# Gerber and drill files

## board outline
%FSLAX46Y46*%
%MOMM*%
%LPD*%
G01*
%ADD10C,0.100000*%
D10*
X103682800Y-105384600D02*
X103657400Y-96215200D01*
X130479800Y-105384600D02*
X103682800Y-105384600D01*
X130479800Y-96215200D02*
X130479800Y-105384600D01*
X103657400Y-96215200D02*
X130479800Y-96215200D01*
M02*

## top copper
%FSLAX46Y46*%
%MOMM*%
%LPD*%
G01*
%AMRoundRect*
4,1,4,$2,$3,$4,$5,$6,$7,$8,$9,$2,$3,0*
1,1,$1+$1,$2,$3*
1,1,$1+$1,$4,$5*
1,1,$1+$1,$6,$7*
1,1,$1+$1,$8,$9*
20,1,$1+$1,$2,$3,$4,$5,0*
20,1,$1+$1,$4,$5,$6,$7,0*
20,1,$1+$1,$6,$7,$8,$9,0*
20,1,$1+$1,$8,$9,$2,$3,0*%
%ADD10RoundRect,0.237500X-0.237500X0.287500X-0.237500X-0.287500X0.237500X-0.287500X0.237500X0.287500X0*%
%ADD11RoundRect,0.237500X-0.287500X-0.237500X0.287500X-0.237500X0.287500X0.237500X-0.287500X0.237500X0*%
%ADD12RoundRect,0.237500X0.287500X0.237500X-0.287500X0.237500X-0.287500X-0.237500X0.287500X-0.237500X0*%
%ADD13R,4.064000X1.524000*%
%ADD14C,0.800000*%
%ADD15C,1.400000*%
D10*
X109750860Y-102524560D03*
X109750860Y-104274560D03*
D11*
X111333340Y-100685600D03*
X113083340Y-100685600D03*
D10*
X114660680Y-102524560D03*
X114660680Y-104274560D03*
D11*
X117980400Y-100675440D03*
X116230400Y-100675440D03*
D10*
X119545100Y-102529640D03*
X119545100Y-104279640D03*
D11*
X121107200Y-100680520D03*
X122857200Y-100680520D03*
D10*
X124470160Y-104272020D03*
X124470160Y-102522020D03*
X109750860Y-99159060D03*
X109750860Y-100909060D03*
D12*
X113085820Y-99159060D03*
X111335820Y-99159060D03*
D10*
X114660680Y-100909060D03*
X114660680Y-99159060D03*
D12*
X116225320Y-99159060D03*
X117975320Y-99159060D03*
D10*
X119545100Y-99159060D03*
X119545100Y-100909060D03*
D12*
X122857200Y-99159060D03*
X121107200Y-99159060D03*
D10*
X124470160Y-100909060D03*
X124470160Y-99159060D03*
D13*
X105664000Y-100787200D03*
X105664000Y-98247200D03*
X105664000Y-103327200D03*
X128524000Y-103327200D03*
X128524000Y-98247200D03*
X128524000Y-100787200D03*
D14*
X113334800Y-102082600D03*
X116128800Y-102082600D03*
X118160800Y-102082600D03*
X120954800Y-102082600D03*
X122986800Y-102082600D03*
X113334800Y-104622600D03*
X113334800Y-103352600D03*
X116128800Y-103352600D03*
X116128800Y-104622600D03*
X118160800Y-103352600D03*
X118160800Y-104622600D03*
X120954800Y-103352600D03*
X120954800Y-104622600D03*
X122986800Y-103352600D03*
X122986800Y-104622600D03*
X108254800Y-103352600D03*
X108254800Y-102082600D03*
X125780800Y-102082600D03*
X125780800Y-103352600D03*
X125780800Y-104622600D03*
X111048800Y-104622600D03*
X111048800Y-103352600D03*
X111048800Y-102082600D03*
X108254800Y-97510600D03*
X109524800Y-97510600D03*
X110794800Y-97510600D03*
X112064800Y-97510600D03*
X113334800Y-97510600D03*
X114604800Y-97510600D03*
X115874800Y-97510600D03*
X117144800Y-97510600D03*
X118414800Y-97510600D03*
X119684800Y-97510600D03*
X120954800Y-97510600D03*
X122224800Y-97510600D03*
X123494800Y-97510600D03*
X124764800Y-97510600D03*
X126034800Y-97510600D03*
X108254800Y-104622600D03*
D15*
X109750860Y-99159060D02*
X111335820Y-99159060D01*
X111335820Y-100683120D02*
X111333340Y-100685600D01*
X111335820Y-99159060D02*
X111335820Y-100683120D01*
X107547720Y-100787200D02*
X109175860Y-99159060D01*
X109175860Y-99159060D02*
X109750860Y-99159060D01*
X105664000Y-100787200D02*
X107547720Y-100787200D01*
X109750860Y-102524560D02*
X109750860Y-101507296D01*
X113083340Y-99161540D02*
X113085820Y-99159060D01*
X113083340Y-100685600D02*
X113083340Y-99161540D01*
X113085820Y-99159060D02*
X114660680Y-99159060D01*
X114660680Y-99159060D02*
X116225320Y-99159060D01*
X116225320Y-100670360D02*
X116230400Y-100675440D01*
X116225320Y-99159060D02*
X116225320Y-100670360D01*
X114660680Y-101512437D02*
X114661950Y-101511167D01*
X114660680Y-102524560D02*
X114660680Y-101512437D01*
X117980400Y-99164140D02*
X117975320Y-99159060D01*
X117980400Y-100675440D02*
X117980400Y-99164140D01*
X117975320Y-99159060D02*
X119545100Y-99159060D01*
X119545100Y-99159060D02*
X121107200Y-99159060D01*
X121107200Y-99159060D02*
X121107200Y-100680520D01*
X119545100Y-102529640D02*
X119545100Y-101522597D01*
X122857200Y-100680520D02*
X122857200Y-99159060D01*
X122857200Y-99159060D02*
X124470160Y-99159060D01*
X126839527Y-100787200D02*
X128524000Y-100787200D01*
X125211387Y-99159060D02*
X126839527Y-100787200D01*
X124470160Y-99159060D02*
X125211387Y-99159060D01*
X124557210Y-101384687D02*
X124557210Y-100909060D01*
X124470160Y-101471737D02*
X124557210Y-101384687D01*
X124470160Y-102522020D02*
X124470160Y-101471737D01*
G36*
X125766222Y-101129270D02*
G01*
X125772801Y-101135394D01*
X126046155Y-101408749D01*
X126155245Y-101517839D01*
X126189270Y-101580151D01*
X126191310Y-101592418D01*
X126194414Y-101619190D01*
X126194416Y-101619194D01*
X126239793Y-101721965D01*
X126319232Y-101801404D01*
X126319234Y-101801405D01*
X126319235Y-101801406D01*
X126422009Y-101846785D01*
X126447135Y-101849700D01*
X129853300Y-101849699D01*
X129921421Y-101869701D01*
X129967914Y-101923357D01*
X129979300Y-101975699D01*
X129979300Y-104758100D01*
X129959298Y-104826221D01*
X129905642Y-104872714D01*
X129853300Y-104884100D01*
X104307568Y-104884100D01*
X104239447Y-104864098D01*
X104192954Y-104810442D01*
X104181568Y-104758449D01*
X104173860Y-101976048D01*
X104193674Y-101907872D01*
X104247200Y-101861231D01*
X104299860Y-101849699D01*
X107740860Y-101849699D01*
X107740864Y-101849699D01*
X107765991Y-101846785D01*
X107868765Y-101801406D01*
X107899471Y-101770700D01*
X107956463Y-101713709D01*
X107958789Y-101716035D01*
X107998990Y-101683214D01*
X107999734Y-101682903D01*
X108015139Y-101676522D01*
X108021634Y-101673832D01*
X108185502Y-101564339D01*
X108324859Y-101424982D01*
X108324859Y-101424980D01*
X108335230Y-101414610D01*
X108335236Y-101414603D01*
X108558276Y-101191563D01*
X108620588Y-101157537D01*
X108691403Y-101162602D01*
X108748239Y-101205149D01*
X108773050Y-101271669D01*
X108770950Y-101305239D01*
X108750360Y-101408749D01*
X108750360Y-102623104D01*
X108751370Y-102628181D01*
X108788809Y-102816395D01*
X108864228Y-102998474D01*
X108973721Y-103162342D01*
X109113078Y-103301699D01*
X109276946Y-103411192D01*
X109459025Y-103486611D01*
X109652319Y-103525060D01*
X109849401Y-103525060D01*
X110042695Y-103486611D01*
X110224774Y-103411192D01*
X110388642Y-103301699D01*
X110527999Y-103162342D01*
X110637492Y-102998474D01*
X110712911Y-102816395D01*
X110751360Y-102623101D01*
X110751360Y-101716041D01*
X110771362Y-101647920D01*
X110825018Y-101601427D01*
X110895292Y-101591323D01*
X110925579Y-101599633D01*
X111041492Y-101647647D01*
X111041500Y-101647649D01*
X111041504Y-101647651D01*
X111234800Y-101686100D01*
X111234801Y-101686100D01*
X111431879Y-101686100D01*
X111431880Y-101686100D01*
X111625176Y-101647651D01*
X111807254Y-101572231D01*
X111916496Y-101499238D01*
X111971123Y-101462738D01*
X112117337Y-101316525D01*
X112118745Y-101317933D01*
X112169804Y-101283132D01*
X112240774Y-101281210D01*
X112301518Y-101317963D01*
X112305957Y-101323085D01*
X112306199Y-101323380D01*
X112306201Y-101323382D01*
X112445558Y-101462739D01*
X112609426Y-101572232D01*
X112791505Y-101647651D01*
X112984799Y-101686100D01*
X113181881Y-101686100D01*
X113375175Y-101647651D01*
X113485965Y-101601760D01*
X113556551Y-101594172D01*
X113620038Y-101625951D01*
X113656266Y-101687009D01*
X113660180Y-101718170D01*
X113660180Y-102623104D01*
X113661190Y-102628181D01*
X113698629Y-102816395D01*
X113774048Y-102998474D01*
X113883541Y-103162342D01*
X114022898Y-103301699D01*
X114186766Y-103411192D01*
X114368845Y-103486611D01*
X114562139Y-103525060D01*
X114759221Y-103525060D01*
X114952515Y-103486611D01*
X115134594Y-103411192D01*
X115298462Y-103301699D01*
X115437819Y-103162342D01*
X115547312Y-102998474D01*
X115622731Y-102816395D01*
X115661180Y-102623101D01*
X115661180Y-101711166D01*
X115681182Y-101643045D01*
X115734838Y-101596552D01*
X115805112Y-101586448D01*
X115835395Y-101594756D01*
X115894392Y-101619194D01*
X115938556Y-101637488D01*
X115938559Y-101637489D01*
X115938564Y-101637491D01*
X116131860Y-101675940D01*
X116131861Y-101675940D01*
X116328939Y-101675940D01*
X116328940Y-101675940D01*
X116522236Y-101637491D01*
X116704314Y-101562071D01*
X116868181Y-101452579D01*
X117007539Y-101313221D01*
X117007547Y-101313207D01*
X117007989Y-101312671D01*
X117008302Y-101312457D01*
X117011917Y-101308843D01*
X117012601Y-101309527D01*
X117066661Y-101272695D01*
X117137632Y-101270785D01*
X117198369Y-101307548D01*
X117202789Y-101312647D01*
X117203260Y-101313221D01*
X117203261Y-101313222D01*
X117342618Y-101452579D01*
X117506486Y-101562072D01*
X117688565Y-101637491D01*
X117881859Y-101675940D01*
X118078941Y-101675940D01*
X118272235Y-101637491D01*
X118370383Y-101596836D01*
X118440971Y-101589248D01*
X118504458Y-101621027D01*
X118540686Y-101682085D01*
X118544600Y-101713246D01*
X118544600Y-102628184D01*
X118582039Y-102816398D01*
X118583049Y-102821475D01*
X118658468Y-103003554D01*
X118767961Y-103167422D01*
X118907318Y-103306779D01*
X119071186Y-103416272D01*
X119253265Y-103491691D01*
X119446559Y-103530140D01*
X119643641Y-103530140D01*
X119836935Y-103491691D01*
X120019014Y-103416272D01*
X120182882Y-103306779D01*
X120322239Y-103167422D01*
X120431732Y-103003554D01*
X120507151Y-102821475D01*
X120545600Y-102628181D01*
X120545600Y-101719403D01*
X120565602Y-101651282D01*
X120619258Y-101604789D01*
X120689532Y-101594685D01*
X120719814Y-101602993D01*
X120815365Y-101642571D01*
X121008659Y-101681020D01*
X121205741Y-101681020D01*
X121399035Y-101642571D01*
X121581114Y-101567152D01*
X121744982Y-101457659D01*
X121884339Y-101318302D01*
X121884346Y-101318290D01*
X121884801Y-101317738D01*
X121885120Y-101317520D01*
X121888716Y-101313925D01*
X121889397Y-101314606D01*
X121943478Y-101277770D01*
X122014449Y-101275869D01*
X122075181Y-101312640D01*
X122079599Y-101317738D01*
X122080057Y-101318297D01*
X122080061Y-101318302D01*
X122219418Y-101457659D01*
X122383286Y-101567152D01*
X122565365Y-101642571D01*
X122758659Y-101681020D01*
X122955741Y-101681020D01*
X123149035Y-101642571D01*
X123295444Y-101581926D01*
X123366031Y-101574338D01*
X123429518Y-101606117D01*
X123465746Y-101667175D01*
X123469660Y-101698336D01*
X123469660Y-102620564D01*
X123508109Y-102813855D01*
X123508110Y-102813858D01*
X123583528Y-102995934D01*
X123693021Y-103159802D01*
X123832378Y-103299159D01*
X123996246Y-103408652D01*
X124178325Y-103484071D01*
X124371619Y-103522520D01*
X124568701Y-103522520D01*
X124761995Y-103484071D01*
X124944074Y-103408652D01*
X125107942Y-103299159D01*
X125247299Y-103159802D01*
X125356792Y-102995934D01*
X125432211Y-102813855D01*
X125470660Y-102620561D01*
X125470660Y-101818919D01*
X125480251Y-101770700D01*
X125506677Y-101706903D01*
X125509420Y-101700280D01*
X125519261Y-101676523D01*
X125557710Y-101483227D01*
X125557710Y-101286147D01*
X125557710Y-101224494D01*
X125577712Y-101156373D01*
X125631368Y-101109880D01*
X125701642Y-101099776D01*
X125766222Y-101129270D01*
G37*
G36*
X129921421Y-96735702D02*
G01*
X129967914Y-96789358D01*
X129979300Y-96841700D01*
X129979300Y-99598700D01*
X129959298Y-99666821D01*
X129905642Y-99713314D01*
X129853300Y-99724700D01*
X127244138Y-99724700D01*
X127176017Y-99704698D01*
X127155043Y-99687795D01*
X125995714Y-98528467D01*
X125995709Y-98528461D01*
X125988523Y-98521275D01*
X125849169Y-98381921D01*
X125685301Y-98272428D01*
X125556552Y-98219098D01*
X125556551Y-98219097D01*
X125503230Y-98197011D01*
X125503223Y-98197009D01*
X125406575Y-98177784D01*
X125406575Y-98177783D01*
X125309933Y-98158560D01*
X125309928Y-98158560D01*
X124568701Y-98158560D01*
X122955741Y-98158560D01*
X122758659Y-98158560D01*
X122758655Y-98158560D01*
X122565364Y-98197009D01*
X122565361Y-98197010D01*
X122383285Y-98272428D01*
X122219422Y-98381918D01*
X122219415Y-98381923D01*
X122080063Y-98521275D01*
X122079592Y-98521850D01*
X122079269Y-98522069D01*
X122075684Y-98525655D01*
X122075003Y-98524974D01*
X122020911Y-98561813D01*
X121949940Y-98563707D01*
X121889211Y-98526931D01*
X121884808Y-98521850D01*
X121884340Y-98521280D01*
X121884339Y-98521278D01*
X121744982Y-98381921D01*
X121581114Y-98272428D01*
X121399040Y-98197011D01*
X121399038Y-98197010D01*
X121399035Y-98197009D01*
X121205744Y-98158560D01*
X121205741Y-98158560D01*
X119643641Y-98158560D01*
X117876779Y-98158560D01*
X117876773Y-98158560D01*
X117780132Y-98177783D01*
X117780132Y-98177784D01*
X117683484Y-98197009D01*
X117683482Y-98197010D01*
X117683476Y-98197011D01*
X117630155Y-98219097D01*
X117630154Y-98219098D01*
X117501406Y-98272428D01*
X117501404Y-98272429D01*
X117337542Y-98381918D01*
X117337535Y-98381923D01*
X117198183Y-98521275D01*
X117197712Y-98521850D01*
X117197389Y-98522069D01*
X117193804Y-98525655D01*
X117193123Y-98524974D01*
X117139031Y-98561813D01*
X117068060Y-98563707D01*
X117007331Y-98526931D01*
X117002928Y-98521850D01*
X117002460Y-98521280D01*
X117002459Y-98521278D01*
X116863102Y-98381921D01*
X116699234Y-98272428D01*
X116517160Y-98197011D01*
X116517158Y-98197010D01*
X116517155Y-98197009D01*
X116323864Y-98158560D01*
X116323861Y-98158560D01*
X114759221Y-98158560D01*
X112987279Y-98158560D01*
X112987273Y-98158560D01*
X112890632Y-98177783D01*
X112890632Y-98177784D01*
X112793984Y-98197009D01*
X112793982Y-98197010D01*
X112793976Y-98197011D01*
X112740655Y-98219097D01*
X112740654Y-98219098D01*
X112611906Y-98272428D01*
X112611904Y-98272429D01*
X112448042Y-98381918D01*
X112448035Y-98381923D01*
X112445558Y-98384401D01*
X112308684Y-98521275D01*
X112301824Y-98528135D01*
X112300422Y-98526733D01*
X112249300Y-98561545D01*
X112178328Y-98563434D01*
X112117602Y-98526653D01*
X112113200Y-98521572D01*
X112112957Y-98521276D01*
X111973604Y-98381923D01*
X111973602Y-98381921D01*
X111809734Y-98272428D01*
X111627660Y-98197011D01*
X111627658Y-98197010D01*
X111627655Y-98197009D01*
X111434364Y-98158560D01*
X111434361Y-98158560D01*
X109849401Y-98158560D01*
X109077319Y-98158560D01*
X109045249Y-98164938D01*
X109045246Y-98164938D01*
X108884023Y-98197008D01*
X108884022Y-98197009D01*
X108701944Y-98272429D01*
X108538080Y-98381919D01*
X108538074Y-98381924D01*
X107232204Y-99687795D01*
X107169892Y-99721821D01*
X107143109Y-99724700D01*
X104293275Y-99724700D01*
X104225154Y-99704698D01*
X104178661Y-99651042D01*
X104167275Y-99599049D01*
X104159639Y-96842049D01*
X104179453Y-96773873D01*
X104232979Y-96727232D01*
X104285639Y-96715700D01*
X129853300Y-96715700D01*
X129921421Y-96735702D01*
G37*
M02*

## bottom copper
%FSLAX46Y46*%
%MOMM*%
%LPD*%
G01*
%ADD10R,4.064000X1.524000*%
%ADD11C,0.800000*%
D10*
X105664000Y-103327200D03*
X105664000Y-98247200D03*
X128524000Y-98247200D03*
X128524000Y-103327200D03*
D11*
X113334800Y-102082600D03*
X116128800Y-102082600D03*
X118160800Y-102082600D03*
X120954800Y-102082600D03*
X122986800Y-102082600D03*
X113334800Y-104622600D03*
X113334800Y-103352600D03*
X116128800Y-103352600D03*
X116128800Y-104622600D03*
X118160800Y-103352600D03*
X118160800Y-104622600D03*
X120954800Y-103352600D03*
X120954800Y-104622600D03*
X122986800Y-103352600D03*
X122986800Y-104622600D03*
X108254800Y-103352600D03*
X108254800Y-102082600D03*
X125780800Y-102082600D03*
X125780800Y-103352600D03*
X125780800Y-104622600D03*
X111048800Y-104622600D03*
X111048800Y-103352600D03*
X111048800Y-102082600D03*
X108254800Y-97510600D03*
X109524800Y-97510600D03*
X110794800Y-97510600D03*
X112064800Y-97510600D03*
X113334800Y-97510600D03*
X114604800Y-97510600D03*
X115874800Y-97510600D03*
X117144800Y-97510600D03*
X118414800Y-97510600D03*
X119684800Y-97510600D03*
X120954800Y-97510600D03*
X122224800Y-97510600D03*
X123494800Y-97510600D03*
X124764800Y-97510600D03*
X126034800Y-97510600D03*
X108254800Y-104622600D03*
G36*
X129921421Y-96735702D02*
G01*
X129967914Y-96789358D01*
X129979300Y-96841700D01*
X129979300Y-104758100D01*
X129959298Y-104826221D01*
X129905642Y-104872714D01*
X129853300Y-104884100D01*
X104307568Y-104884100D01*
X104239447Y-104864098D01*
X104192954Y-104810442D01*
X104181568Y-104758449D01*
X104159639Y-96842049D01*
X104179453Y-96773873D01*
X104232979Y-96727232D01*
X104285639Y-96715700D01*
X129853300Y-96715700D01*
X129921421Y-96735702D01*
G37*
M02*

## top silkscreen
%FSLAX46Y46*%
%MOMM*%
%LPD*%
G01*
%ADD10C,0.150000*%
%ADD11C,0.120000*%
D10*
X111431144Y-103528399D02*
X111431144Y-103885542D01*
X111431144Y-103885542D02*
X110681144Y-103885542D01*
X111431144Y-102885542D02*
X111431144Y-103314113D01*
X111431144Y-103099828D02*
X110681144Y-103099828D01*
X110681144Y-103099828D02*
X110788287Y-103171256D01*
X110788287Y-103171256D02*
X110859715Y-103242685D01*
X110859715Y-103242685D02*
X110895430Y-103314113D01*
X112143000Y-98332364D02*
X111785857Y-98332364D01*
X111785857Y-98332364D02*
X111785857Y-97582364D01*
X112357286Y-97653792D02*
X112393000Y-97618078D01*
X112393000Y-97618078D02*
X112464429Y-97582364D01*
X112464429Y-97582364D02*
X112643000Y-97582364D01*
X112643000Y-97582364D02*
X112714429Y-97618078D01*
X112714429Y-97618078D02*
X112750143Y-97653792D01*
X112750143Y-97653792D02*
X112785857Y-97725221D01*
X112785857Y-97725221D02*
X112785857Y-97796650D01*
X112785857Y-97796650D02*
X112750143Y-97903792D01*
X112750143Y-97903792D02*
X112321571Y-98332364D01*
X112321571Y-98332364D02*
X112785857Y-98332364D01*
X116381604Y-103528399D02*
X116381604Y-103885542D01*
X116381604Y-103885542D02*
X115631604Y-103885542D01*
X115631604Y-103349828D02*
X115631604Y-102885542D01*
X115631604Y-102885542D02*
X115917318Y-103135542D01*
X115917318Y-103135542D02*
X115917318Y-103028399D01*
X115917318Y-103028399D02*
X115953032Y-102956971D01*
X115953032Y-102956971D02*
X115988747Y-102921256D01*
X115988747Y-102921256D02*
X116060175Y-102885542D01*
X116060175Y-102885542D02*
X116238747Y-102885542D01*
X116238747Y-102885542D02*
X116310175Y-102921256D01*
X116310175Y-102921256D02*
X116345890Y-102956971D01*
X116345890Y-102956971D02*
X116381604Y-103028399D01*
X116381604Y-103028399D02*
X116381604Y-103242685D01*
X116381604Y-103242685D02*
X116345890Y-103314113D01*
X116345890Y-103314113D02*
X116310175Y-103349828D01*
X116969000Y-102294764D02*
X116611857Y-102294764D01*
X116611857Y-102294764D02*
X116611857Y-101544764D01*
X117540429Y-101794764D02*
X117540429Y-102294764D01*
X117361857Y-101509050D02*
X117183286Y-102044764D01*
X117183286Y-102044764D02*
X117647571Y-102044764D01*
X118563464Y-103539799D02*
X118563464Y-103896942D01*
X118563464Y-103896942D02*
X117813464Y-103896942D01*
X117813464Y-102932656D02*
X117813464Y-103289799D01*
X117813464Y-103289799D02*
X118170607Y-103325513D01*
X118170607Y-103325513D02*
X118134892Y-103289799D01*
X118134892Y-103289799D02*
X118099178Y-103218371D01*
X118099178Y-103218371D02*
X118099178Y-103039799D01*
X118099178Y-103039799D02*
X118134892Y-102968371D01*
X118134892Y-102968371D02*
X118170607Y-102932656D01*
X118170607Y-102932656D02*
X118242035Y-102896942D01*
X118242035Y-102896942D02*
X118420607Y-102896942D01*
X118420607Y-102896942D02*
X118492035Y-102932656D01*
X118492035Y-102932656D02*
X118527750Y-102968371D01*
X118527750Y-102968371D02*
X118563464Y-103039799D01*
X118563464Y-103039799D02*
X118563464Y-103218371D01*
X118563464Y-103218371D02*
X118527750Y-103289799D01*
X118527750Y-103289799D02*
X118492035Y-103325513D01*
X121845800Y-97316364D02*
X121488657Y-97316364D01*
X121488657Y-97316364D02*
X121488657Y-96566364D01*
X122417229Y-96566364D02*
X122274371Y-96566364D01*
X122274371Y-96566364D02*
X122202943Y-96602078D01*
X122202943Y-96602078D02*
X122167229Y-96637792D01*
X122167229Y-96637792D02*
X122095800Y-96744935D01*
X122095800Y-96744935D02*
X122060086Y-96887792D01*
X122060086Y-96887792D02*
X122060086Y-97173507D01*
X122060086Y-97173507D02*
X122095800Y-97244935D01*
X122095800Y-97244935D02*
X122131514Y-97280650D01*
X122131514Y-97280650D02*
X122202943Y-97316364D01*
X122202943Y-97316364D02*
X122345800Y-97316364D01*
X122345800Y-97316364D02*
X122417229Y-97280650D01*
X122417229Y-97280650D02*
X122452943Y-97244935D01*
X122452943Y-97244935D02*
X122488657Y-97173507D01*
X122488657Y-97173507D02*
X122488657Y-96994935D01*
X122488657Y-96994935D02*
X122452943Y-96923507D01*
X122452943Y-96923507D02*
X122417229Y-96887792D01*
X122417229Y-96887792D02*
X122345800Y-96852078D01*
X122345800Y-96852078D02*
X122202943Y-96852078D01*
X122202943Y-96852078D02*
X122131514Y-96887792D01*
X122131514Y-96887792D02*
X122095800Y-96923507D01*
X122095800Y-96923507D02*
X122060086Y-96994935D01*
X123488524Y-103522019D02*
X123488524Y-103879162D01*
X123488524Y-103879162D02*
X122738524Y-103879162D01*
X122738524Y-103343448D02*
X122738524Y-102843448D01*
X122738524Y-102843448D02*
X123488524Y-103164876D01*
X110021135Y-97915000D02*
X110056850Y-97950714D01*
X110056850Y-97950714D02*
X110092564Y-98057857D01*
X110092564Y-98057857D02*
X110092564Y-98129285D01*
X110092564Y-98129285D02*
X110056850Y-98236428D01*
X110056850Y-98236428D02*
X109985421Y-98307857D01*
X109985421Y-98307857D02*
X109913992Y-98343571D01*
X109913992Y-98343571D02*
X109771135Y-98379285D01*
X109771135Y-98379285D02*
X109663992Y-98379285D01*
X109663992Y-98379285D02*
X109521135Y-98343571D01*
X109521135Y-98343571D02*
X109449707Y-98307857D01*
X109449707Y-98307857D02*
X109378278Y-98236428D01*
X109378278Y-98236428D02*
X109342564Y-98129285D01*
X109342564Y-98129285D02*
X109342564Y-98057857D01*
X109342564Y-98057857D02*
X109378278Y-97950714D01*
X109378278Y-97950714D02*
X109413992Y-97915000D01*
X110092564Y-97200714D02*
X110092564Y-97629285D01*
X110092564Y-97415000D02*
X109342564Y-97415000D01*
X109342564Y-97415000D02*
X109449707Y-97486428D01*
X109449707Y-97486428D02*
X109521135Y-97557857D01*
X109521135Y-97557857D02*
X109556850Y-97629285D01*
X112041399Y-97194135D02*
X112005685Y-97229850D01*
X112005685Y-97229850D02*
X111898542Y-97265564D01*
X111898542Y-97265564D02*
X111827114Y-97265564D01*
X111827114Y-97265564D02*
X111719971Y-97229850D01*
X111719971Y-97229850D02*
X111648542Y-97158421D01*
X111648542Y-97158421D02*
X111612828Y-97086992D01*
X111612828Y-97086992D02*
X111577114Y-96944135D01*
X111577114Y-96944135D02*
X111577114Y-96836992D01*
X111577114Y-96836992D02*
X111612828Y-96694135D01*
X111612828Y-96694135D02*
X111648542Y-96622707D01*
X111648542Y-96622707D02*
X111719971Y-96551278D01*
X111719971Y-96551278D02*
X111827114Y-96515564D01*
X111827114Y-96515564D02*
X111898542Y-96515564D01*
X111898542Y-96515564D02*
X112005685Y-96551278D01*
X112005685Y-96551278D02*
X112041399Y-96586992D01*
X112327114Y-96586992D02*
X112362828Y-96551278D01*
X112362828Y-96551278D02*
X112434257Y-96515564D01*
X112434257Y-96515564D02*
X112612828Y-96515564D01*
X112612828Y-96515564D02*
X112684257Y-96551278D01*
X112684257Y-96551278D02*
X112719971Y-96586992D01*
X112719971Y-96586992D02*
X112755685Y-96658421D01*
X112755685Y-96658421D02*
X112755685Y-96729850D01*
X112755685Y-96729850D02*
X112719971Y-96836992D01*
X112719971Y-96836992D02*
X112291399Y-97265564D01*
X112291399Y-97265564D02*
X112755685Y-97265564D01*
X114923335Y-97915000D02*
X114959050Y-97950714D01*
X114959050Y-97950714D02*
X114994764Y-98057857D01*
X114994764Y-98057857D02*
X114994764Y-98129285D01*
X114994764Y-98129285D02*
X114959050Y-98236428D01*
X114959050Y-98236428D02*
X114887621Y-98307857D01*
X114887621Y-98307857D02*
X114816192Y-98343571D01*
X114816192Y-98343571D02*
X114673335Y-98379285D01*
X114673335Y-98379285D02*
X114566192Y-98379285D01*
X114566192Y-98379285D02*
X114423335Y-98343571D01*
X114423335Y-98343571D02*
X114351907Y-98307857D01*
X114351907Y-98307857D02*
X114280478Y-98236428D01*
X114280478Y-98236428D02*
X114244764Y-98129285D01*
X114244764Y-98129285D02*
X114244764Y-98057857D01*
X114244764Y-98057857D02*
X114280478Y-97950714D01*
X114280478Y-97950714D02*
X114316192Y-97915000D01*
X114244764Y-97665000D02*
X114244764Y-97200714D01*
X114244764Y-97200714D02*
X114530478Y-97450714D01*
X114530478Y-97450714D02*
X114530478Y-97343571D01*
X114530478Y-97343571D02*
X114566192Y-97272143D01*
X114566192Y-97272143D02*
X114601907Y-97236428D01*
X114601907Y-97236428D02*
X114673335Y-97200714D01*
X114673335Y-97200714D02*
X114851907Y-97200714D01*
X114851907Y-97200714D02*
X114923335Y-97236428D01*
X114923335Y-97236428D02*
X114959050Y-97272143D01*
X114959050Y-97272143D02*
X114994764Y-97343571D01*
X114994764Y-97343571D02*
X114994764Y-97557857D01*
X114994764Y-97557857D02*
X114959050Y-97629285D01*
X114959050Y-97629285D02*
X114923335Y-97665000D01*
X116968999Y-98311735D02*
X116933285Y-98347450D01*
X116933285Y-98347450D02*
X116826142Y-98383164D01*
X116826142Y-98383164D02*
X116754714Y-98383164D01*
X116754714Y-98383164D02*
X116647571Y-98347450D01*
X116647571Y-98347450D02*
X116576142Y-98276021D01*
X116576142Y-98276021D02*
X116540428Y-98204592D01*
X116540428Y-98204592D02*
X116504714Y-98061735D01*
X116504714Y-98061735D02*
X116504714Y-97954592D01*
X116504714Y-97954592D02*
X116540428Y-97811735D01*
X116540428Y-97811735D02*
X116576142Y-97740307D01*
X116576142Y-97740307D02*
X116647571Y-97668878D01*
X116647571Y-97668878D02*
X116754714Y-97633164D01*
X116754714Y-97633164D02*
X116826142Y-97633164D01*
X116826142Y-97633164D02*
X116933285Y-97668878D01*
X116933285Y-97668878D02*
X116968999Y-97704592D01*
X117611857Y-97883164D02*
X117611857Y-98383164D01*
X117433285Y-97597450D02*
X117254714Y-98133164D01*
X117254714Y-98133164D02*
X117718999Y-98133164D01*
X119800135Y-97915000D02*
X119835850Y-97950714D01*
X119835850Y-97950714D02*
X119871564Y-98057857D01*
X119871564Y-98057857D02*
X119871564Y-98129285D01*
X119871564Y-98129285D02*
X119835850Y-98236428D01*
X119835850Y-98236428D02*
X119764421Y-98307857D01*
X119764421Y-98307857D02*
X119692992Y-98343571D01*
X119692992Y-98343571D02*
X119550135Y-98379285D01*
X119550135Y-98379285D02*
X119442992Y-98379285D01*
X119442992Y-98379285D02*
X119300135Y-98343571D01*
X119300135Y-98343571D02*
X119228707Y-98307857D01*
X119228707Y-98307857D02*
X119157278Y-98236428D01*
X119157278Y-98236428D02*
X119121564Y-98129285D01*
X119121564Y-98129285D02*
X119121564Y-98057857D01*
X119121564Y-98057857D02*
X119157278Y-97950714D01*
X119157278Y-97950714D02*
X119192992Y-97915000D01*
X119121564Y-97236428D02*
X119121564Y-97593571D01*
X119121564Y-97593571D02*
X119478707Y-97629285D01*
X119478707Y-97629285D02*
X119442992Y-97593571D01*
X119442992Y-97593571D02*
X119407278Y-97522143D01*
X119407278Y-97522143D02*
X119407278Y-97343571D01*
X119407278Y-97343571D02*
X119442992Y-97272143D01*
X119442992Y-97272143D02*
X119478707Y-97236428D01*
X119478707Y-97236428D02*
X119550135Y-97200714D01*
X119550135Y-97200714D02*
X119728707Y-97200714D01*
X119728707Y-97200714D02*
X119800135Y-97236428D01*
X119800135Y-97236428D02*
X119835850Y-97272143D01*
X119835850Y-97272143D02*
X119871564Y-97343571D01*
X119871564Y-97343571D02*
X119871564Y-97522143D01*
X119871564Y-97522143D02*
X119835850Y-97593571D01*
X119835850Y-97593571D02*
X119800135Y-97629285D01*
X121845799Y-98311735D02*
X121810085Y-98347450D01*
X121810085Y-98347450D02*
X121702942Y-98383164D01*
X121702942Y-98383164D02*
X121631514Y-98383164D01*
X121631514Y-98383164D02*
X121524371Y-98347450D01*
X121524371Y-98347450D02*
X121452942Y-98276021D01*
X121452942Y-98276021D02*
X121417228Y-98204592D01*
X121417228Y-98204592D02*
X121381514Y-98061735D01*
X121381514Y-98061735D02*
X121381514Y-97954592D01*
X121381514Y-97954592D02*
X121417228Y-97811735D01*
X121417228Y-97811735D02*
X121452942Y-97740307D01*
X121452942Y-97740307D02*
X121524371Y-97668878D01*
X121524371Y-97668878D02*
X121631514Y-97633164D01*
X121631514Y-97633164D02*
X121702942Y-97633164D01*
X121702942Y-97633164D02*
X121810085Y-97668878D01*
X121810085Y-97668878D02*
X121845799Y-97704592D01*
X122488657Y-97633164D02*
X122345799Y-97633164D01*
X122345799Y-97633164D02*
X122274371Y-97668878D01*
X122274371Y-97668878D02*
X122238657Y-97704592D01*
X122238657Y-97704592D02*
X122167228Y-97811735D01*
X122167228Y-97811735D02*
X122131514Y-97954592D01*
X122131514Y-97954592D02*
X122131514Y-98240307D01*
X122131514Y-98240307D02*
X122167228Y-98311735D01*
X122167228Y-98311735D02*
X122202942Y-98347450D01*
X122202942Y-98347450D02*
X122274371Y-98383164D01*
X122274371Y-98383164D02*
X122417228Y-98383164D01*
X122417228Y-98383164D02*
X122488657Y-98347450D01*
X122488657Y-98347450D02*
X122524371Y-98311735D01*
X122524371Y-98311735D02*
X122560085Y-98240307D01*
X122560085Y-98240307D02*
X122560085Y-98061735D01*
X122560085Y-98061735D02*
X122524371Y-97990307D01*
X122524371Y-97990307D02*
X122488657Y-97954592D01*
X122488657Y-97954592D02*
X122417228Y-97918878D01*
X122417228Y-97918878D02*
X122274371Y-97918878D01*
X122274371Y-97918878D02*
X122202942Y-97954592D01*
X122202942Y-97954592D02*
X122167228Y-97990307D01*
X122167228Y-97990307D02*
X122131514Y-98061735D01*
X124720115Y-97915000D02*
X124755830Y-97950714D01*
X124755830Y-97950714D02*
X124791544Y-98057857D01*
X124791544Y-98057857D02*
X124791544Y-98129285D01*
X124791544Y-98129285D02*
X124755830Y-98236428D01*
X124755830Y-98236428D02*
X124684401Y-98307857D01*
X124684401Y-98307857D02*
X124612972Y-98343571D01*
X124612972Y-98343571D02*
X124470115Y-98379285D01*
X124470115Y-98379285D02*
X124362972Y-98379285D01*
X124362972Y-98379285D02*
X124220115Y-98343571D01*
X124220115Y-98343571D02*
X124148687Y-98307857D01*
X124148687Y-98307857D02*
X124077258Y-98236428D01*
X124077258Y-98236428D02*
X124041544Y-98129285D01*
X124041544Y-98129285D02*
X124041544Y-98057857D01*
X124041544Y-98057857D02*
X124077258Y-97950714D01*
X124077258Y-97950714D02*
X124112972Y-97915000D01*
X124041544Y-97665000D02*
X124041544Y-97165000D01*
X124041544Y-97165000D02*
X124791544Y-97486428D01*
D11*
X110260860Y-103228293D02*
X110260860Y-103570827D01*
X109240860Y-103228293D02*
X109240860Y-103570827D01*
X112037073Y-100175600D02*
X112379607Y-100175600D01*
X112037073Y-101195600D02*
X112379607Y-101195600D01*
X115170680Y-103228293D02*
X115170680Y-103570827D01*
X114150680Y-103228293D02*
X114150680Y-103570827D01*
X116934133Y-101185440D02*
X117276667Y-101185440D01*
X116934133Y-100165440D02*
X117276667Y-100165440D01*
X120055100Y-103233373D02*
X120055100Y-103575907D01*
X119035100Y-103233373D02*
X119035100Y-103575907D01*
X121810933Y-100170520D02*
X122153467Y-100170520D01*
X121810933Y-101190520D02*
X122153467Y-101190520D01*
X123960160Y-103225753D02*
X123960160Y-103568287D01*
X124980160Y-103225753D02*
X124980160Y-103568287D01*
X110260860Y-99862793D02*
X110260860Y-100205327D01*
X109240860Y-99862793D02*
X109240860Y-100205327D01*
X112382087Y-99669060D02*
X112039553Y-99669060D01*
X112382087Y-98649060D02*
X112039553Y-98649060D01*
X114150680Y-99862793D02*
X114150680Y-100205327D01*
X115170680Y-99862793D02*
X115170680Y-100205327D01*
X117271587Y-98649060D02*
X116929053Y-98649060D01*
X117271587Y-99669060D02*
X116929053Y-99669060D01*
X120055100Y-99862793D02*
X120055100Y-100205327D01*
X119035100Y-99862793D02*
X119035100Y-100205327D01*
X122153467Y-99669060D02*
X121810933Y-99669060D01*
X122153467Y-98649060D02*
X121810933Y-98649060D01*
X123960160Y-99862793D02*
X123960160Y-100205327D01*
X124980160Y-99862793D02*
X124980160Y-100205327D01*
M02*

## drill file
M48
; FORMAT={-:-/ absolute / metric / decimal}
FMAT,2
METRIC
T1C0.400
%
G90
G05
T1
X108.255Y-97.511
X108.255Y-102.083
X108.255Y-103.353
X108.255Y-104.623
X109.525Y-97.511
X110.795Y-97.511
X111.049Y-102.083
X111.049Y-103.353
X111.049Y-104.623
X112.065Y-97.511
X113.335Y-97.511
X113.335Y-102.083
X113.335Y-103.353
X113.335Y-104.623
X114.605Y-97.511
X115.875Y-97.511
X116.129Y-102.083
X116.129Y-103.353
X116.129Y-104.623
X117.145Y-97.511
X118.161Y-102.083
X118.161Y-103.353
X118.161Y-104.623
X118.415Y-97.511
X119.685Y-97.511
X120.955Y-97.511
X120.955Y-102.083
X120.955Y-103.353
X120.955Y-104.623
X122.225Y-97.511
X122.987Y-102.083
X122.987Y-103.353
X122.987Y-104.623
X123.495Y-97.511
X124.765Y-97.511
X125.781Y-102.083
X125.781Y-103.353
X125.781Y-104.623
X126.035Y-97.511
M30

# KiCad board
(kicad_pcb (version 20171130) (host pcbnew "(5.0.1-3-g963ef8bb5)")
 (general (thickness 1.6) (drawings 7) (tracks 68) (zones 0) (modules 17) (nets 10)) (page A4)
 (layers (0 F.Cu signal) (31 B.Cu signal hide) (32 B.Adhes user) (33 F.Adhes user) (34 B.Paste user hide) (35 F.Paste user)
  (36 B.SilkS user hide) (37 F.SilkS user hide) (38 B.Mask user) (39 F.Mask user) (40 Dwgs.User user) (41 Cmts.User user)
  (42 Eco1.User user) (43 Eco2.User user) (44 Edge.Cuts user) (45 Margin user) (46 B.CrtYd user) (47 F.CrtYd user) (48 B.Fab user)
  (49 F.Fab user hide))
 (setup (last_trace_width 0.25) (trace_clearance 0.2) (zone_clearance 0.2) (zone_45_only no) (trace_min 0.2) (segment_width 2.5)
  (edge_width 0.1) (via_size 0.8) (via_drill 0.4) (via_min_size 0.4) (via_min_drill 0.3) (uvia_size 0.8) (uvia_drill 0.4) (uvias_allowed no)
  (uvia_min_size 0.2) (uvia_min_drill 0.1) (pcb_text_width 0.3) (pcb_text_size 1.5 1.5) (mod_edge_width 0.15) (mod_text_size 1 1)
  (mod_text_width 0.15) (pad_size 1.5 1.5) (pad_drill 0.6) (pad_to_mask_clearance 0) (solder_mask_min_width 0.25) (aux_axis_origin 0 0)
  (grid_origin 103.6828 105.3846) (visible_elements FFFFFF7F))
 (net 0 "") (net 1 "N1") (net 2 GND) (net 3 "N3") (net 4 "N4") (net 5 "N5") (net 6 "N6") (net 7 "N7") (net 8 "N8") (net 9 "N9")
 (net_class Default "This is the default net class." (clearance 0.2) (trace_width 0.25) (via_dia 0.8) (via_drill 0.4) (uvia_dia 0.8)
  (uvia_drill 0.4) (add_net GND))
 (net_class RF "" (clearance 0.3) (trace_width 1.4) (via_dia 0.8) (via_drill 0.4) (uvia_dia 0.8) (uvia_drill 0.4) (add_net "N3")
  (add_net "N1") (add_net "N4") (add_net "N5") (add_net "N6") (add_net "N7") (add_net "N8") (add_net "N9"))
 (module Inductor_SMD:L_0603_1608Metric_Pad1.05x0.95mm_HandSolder (layer F.Cu) (at 109.75086 103.39956 270)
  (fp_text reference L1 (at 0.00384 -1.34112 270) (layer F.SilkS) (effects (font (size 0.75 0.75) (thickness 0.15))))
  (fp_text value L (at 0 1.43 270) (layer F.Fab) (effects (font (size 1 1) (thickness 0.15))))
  (fp_line (start -0.171267 -0.51) (end 0.171267 -0.51) (layer F.SilkS) (width 0.12))
  (fp_line (start -0.171267 0.51) (end 0.171267 0.51) (layer F.SilkS) (width 0.12))
  (pad 1 smd roundrect (at -0.875 0 270) (size 1.05 0.95) (layers F.Cu F.Paste F.Mask) (roundrect_rratio 0.25) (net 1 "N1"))
  (pad 2 smd roundrect (at 0.875 0 270) (size 1.05 0.95) (layers F.Cu F.Paste F.Mask) (roundrect_rratio 0.25) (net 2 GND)))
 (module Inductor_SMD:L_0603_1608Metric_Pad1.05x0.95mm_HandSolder (layer F.Cu) (at 112.20834 100.6856)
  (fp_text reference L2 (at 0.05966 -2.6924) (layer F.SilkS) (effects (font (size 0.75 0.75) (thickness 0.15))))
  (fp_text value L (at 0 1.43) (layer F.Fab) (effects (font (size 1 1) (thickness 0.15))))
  (fp_line (start -0.171267 -0.51) (end 0.171267 -0.51) (layer F.SilkS) (width 0.12))
  (fp_line (start -0.171267 0.51) (end 0.171267 0.51) (layer F.SilkS) (width 0.12))
  (pad 1 smd roundrect (at -0.875 0) (size 1.05 0.95) (layers F.Cu F.Paste F.Mask) (roundrect_rratio 0.25) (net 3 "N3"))
  (pad 2 smd roundrect (at 0.875 0) (size 1.05 0.95) (layers F.Cu F.Paste F.Mask) (roundrect_rratio 0.25) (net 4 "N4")))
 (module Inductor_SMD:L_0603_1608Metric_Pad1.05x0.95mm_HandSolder (layer F.Cu) (at 114.66068 103.39956 270)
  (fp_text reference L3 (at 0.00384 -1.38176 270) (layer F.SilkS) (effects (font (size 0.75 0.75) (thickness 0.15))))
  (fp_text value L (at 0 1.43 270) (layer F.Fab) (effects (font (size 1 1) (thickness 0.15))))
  (fp_line (start -0.171267 -0.51) (end 0.171267 -0.51) (layer F.SilkS) (width 0.12))
  (fp_line (start -0.171267 0.51) (end 0.171267 0.51) (layer F.SilkS) (width 0.12))
  (pad 1 smd roundrect (at -0.875 0 270) (size 1.05 0.95) (layers F.Cu F.Paste F.Mask) (roundrect_rratio 0.25) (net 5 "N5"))
  (pad 2 smd roundrect (at 0.875 0 270) (size 1.05 0.95) (layers F.Cu F.Paste F.Mask) (roundrect_rratio 0.25) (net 2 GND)))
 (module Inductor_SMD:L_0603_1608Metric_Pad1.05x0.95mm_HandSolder (layer F.Cu) (at 117.1054 100.67544)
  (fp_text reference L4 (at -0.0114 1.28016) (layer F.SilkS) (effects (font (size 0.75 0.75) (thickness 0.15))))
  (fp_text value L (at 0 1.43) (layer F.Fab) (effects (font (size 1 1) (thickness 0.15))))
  (fp_line (start -0.171267 0.51) (end 0.171267 0.51) (layer F.SilkS) (width 0.12))
  (fp_line (start -0.171267 -0.51) (end 0.171267 -0.51) (layer F.SilkS) (width 0.12))
  (pad 2 smd roundrect (at 0.875 0) (size 1.05 0.95) (layers F.Cu F.Paste F.Mask) (roundrect_rratio 0.25) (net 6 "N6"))
  (pad 1 smd roundrect (at -0.875 0) (size 1.05 0.95) (layers F.Cu F.Paste F.Mask) (roundrect_rratio 0.25) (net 4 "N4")))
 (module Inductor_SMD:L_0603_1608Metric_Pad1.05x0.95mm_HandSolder (layer F.Cu) (at 119.5451 103.40464 270)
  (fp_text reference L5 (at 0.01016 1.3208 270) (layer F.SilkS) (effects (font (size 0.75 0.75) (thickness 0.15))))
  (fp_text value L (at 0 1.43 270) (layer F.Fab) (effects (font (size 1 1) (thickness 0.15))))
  (fp_line (start -0.171267 -0.51) (end 0.171267 -0.51) (layer F.SilkS) (width 0.12))
  (fp_line (start -0.171267 0.51) (end 0.171267 0.51) (layer F.SilkS) (width 0.12))
  (pad 1 smd roundrect (at -0.875 0 270) (size 1.05 0.95) (layers F.Cu F.Paste F.Mask) (roundrect_rratio 0.25) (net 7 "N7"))
  (pad 2 smd roundrect (at 0.875 0 270) (size 1.05 0.95) (layers F.Cu F.Paste F.Mask) (roundrect_rratio 0.25) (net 2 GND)))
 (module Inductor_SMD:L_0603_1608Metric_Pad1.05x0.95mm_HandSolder (layer F.Cu) (at 121.9822 100.68052)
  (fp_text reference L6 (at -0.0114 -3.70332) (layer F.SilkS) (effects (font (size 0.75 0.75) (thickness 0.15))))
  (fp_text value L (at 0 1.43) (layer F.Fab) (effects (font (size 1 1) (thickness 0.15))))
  (fp_line (start -0.171267 -0.51) (end 0.171267 -0.51) (layer F.SilkS) (width 0.12))
  (fp_line (start -0.171267 0.51) (end 0.171267 0.51) (layer F.SilkS) (width 0.12))
  (pad 1 smd roundrect (at -0.875 0) (size 1.05 0.95) (layers F.Cu F.Paste F.Mask) (roundrect_rratio 0.25) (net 6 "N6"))
  (pad 2 smd roundrect (at 0.875 0) (size 1.05 0.95) (layers F.Cu F.Paste F.Mask) (roundrect_rratio 0.25) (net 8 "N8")))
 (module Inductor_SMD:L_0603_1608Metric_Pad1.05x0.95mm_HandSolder (layer F.Cu) (at 124.47016 103.39702 270)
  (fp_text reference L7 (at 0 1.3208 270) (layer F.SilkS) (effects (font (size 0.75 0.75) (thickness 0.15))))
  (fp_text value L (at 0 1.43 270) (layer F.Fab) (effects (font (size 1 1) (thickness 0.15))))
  (fp_line (start -0.171267 0.51) (end 0.171267 0.51) (layer F.SilkS) (width 0.12))
  (fp_line (start -0.171267 -0.51) (end 0.171267 -0.51) (layer F.SilkS) (width 0.12))
  (pad 2 smd roundrect (at 0.875 0 270) (size 1.05 0.95) (layers F.Cu F.Paste F.Mask) (roundrect_rratio 0.25) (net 2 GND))
  (pad 1 smd roundrect (at -0.875 0 270) (size 1.05 0.95) (layers F.Cu F.Paste F.Mask) (roundrect_rratio 0.25) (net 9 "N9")))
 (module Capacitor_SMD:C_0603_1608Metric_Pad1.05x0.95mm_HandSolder (layer F.Cu) (at 109.75086 100.03406 270)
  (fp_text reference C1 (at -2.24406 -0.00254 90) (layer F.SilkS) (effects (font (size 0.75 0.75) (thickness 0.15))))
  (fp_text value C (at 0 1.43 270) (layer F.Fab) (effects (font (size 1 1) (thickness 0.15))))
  (fp_line (start -0.171267 -0.51) (end 0.171267 -0.51) (layer F.SilkS) (width 0.12))
  (fp_line (start -0.171267 0.51) (end 0.171267 0.51) (layer F.SilkS) (width 0.12))
  (pad 1 smd roundrect (at -0.875 0 270) (size 1.05 0.95) (layers F.Cu F.Paste F.Mask) (roundrect_rratio 0.25) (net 3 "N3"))
  (pad 2 smd roundrect (at 0.875 0 270) (size 1.05 0.95) (layers F.Cu F.Paste F.Mask) (roundrect_rratio 0.25) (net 1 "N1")))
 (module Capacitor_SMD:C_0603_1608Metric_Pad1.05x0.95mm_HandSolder (layer F.Cu) (at 112.21082 99.15906 180)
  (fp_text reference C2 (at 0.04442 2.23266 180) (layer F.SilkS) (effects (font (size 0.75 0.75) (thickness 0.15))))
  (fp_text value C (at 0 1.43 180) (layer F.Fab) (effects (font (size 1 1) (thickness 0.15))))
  (fp_line (start -0.171267 -0.51) (end 0.171267 -0.51) (layer F.SilkS) (width 0.12))
  (fp_line (start -0.171267 0.51) (end 0.171267 0.51) (layer F.SilkS) (width 0.12))
  (pad 1 smd roundrect (at -0.875 0 180) (size 1.05 0.95) (layers F.Cu F.Paste F.Mask) (roundrect_rratio 0.25) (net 4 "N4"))
  (pad 2 smd roundrect (at 0.875 0 180) (size 1.05 0.95) (layers F.Cu F.Paste F.Mask) (roundrect_rratio 0.25) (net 3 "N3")))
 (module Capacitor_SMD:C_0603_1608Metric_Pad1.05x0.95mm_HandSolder (layer F.Cu) (at 114.66068 100.03406 270)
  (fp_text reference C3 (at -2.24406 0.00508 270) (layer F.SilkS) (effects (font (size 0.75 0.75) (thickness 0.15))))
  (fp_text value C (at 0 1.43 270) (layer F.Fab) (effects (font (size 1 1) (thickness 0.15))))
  (fp_line (start -0.171267 0.51) (end 0.171267 0.51) (layer F.SilkS) (width 0.12))
  (fp_line (start -0.171267 -0.51) (end 0.171267 -0.51) (layer F.SilkS) (width 0.12))
  (pad 2 smd roundrect (at 0.875 0 270) (size 1.05 0.95) (layers F.Cu F.Paste F.Mask) (roundrect_rratio 0.25) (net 5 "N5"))
  (pad 1 smd roundrect (at -0.875 0 270) (size 1.05 0.95) (layers F.Cu F.Paste F.Mask) (roundrect_rratio 0.25) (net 4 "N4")))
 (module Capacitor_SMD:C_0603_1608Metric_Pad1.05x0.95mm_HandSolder (layer F.Cu) (at 117.10032 99.15906 180)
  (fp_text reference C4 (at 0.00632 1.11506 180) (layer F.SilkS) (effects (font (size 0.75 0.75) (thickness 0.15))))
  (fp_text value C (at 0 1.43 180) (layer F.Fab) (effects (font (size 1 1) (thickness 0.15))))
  (fp_line (start -0.171267 0.51) (end 0.171267 0.51) (layer F.SilkS) (width 0.12))
  (fp_line (start -0.171267 -0.51) (end 0.171267 -0.51) (layer F.SilkS) (width 0.12))
  (pad 2 smd roundrect (at 0.875 0 180) (size 1.05 0.95) (layers F.Cu F.Paste F.Mask) (roundrect_rratio 0.25) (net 4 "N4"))
  (pad 1 smd roundrect (at -0.875 0 180) (size 1.05 0.95) (layers F.Cu F.Paste F.Mask) (roundrect_rratio 0.25) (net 6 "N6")))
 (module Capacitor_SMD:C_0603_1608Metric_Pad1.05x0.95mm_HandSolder (layer F.Cu) (at 119.5451 100.03406 270)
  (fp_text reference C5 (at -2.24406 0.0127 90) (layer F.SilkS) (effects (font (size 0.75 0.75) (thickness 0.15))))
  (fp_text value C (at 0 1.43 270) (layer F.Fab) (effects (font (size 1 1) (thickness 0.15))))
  (fp_line (start -0.171267 -0.51) (end 0.171267 -0.51) (layer F.SilkS) (width 0.12))
  (fp_line (start -0.171267 0.51) (end 0.171267 0.51) (layer F.SilkS) (width 0.12))
  (pad 1 smd roundrect (at -0.875 0 270) (size 1.05 0.95) (layers F.Cu F.Paste F.Mask) (roundrect_rratio 0.25) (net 6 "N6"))
  (pad 2 smd roundrect (at 0.875 0 270) (size 1.05 0.95) (layers F.Cu F.Paste F.Mask) (roundrect_rratio 0.25) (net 7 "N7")))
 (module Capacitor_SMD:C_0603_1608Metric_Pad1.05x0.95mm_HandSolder (layer F.Cu) (at 121.9822 99.15906 180)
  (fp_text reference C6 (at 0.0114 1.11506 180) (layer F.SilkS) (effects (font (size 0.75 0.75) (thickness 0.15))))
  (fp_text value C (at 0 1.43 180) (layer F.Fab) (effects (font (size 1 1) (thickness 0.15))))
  (fp_line (start -0.171267 -0.51) (end 0.171267 -0.51) (layer F.SilkS) (width 0.12))
  (fp_line (start -0.171267 0.51) (end 0.171267 0.51) (layer F.SilkS) (width 0.12))
  (pad 1 smd roundrect (at -0.875 0 180) (size 1.05 0.95) (layers F.Cu F.Paste F.Mask) (roundrect_rratio 0.25) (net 8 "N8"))
  (pad 2 smd roundrect (at 0.875 0 180) (size 1.05 0.95) (layers F.Cu F.Paste F.Mask) (roundrect_rratio 0.25) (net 6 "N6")))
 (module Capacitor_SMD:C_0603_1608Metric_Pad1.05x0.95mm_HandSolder (layer F.Cu) (at 124.47016 100.03406 270)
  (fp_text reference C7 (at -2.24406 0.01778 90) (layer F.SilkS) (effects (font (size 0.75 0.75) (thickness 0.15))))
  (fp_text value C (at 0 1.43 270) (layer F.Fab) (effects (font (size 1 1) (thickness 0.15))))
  (fp_line (start -0.171267 0.51) (end 0.171267 0.51) (layer F.SilkS) (width 0.12))
  (fp_line (start -0.171267 -0.51) (end 0.171267 -0.51) (layer F.SilkS) (width 0.12))
  (pad 2 smd roundrect (at 0.875 0 270) (size 1.05 0.95) (layers F.Cu F.Paste F.Mask) (roundrect_rratio 0.25) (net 9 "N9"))
  (pad 1 smd roundrect (at -0.875 0 270) (size 1.05 0.95) (layers F.Cu F.Paste F.Mask) (roundrect_rratio 0.25) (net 8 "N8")))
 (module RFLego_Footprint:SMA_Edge (layer F.Cu) (at 103.632 100.7872)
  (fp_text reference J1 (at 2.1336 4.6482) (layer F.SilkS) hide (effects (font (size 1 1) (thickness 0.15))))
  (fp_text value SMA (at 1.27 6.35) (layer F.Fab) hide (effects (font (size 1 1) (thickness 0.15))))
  (pad 1 smd rect (at 2.032 0) (size 4.064 1.524) (layers F.Cu F.Mask) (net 3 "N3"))
  (pad 2 smd rect (at 2.032 -2.54) (size 4.064 1.524) (layers F.Cu F.Mask) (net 2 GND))
  (pad 2 smd rect (at 2.032 2.54) (size 4.064 1.524) (layers B.Cu B.Mask) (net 2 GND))
  (pad 2 smd rect (at 2.032 -2.54) (size 4.064 1.524) (layers B.Cu B.Mask) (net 2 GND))
  (pad 2 smd rect (at 2.032 2.54) (size 4.064 1.524) (layers F.Cu F.Mask) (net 2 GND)))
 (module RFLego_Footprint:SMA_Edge (layer F.Cu) (at 126.492 100.7872)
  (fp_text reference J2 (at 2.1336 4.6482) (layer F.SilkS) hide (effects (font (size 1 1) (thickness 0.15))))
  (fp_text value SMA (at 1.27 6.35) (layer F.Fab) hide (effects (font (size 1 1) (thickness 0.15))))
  (pad 2 smd rect (at 2.032 2.54) (size 4.064 1.524) (layers F.Cu F.Mask) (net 2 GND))
  (pad 2 smd rect (at 2.032 -2.54) (size 4.064 1.524) (layers B.Cu B.Mask) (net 2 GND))
  (pad 2 smd rect (at 2.032 2.54) (size 4.064 1.524) (layers B.Cu B.Mask) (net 2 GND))
  (pad 2 smd rect (at 2.032 -2.54) (size 4.064 1.524) (layers F.Cu F.Mask) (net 2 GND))
  (pad 1 smd rect (at 2.032 0) (size 4.064 1.524) (layers F.Cu F.Mask) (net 8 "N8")))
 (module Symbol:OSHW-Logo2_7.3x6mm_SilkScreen (layer B.Cu) (at 111.00816 102.235 180)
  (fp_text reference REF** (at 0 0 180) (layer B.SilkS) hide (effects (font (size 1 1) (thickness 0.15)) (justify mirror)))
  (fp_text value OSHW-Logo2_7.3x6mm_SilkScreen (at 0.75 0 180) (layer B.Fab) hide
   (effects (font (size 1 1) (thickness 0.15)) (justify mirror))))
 (gr_line (start 103.6828 105.3846) (end 103.6574 96.2152) (layer Edge.Cuts) (width 0.1))
 (gr_line (start 130.4798 105.3846) (end 103.6828 105.3846) (layer Edge.Cuts) (width 0.1))
 (gr_line (start 130.4798 96.2152) (end 130.4798 105.3846) (layer Edge.Cuts) (width 0.1))
 (gr_line (start 103.6574 96.2152) (end 130.4798 96.2152) (layer Edge.Cuts) (width 0.1))
 (via (at 113.3348 102.0826) (size 0.8) (drill 0.4) (layers F.Cu B.Cu) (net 2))
 (via (at 116.1288 102.0826) (size 0.8) (drill 0.4) (layers F.Cu B.Cu) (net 2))
 (via (at 118.1608 102.0826) (size 0.8) (drill 0.4) (layers F.Cu B.Cu) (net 2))
 (via (at 120.9548 102.0826) (size 0.8) (drill 0.4) (layers F.Cu B.Cu) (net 2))
 (via (at 122.9868 102.0826) (size 0.8) (drill 0.4) (layers F.Cu B.Cu) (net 2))
 (via (at 113.3348 104.6226) (size 0.8) (drill 0.4) (layers F.Cu B.Cu) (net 2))
 (via (at 113.3348 103.3526) (size 0.8) (drill 0.4) (layers F.Cu B.Cu) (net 2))
 (via (at 116.1288 103.3526) (size 0.8) (drill 0.4) (layers F.Cu B.Cu) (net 2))
 (via (at 116.1288 104.6226) (size 0.8) (drill 0.4) (layers F.Cu B.Cu) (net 2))
 (via (at 118.1608 103.3526) (size 0.8) (drill 0.4) (layers F.Cu B.Cu) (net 2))
 (via (at 118.1608 104.6226) (size 0.8) (drill 0.4) (layers F.Cu B.Cu) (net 2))
 (via (at 120.9548 103.3526) (size 0.8) (drill 0.4) (layers F.Cu B.Cu) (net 2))
 (via (at 120.9548 104.6226) (size 0.8) (drill 0.4) (layers F.Cu B.Cu) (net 2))
 (via (at 122.9868 103.3526) (size 0.8) (drill 0.4) (layers F.Cu B.Cu) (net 2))
 (via (at 122.9868 104.6226) (size 0.8) (drill 0.4) (layers F.Cu B.Cu) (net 2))
 (via (at 108.2548 103.3526) (size 0.8) (drill 0.4) (layers F.Cu B.Cu) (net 2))
 (via (at 108.2548 102.0826) (size 0.8) (drill 0.4) (layers F.Cu B.Cu) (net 2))
 (via (at 125.7808 102.0826) (size 0.8) (drill 0.4) (layers F.Cu B.Cu) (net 2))
 (via (at 125.7808 103.3526) (size 0.8) (drill 0.4) (layers F.Cu B.Cu) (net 2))
 (via (at 125.7808 104.6226) (size 0.8) (drill 0.4) (layers F.Cu B.Cu) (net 2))
 (via (at 111.0488 104.6226) (size 0.8) (drill 0.4) (layers F.Cu B.Cu) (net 2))
 (via (at 111.0488 103.3526) (size 0.8) (drill 0.4) (layers F.Cu B.Cu) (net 2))
 (via (at 111.0488 102.0826) (size 0.8) (drill 0.4) (layers F.Cu B.Cu) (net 2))
 (segment (start 109.75086 99.15906) (end 111.33582 99.15906) (width 1.4) (layer F.Cu) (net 3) (status 30))
 (segment (start 111.33582 100.68312) (end 111.33334 100.6856) (width 1.4) (layer F.Cu) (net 3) (status 30))
 (segment (start 111.33582 99.15906) (end 111.33582 100.68312) (width 1.4) (layer F.Cu) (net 3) (status 30))
 (segment (start 107.54772 100.7872) (end 109.17586 99.15906) (width 1.4) (layer F.Cu) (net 3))
 (segment (start 109.17586 99.15906) (end 109.75086 99.15906) (width 1.4) (layer F.Cu) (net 3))
 (segment (start 105.664 100.7872) (end 107.54772 100.7872) (width 1.4) (layer F.Cu) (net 3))
 (segment (start 109.75086 102.52456) (end 109.75086 101.507296) (width 1.4) (layer F.Cu) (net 1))
 (segment (start 113.08334 99.16154) (end 113.08582 99.15906) (width 1.4) (layer F.Cu) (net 4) (status 30))
 (segment (start 113.08334 100.6856) (end 113.08334 99.16154) (width 1.4) (layer F.Cu) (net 4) (status 30))
 (segment (start 113.08582 99.15906) (end 114.66068 99.15906) (width 1.4) (layer F.Cu) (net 4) (status 30))
 (segment (start 114.66068 99.15906) (end 116.22532 99.15906) (width 1.4) (layer F.Cu) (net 4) (status 30))
 (segment (start 116.22532 100.67036) (end 116.2304 100.67544) (width 1.4) (layer F.Cu) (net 4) (status 30))
 (segment (start 116.22532 99.15906) (end 116.22532 100.67036) (width 1.4) (layer F.Cu) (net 4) (status 30))
 (segment (start 114.66068 101.512437) (end 114.66195 101.511167) (width 1.4) (layer F.Cu) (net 5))
 (segment (start 114.66068 102.52456) (end 114.66068 101.512437) (width 1.4) (layer F.Cu) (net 5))
 (segment (start 117.9804 99.16414) (end 117.97532 99.15906) (width 1.4) (layer F.Cu) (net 6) (status 30))
 (segment (start 117.9804 100.67544) (end 117.9804 99.16414) (width 1.4) (layer F.Cu) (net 6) (status 30))
 (segment (start 117.97532 99.15906) (end 119.5451 99.15906) (width 1.4) (layer F.Cu) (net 6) (status 30))
 (segment (start 119.5451 99.15906) (end 121.1072 99.15906) (width 1.4) (layer F.Cu) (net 6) (status 30))
 (segment (start 121.1072 99.15906) (end 121.1072 100.68052) (width 1.4) (layer F.Cu) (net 6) (status 30))
 (segment (start 119.5451 102.52964) (end 119.5451 101.522597) (width 1.4) (layer F.Cu) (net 7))
 (segment (start 122.8572 100.68052) (end 122.8572 99.15906) (width 1.4) (layer F.Cu) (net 8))
 (segment (start 122.8572 99.15906) (end 124.47016 99.15906) (width 1.4) (layer F.Cu) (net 8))
 (segment (start 126.839527 100.7872) (end 128.524 100.7872) (width 1.4) (layer F.Cu) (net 8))
 (segment (start 125.211387 99.15906) (end 126.839527 100.7872) (width 1.4) (layer F.Cu) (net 8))
 (segment (start 124.47016 99.15906) (end 125.211387 99.15906) (width 1.4) (layer F.Cu) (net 8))
 (segment (start 124.55721 101.384687) (end 124.55721 100.90906) (width 1.4) (layer F.Cu) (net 9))
 (segment (start 124.47016 101.471737) (end 124.55721 101.384687) (width 1.4) (layer F.Cu) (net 9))
 (segment (start 124.47016 102.52202) (end 124.47016 101.471737) (width 1.4) (layer F.Cu) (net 9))
 (via (at 108.2548 97.5106) (size 0.8) (drill 0.4) (layers F.Cu B.Cu) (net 2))
 (via (at 109.5248 97.5106) (size 0.8) (drill 0.4) (layers F.Cu B.Cu) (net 2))
 (via (at 110.7948 97.5106) (size 0.8) (drill 0.4) (layers F.Cu B.Cu) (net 2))
 (via (at 112.0648 97.5106) (size 0.8) (drill 0.4) (layers F.Cu B.Cu) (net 2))
 (via (at 113.3348 97.5106) (size 0.8) (drill 0.4) (layers F.Cu B.Cu) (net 2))
 (via (at 114.6048 97.5106) (size 0.8) (drill 0.4) (layers F.Cu B.Cu) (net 2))
 (via (at 115.8748 97.5106) (size 0.8) (drill 0.4) (layers F.Cu B.Cu) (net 2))
 (via (at 117.1448 97.5106) (size 0.8) (drill 0.4) (layers F.Cu B.Cu) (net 2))
 (via (at 118.4148 97.5106) (size 0.8) (drill 0.4) (layers F.Cu B.Cu) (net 2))
 (via (at 119.6848 97.5106) (size 0.8) (drill 0.4) (layers F.Cu B.Cu) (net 2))
 (via (at 120.9548 97.5106) (size 0.8) (drill 0.4) (layers F.Cu B.Cu) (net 2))
 (via (at 122.2248 97.5106) (size 0.8) (drill 0.4) (layers F.Cu B.Cu) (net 2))
 (via (at 123.4948 97.5106) (size 0.8) (drill 0.4) (layers F.Cu B.Cu) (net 2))
 (via (at 124.7648 97.5106) (size 0.8) (drill 0.4) (layers F.Cu B.Cu) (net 2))
 (via (at 126.0348 97.5106) (size 0.8) (drill 0.4) (layers F.Cu B.Cu) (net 2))
 (via (at 108.2548 104.6226) (size 0.8) (drill 0.4) (layers F.Cu B.Cu) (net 2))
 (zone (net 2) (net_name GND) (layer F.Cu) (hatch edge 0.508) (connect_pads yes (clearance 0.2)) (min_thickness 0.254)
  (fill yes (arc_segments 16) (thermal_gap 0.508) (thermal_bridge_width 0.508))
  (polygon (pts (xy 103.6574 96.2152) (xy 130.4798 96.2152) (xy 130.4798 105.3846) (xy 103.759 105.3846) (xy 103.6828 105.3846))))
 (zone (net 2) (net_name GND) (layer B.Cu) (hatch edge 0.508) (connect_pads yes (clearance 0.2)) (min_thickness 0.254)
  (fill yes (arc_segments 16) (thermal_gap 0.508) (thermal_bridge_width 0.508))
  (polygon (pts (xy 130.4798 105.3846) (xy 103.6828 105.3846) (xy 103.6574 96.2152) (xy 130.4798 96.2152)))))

